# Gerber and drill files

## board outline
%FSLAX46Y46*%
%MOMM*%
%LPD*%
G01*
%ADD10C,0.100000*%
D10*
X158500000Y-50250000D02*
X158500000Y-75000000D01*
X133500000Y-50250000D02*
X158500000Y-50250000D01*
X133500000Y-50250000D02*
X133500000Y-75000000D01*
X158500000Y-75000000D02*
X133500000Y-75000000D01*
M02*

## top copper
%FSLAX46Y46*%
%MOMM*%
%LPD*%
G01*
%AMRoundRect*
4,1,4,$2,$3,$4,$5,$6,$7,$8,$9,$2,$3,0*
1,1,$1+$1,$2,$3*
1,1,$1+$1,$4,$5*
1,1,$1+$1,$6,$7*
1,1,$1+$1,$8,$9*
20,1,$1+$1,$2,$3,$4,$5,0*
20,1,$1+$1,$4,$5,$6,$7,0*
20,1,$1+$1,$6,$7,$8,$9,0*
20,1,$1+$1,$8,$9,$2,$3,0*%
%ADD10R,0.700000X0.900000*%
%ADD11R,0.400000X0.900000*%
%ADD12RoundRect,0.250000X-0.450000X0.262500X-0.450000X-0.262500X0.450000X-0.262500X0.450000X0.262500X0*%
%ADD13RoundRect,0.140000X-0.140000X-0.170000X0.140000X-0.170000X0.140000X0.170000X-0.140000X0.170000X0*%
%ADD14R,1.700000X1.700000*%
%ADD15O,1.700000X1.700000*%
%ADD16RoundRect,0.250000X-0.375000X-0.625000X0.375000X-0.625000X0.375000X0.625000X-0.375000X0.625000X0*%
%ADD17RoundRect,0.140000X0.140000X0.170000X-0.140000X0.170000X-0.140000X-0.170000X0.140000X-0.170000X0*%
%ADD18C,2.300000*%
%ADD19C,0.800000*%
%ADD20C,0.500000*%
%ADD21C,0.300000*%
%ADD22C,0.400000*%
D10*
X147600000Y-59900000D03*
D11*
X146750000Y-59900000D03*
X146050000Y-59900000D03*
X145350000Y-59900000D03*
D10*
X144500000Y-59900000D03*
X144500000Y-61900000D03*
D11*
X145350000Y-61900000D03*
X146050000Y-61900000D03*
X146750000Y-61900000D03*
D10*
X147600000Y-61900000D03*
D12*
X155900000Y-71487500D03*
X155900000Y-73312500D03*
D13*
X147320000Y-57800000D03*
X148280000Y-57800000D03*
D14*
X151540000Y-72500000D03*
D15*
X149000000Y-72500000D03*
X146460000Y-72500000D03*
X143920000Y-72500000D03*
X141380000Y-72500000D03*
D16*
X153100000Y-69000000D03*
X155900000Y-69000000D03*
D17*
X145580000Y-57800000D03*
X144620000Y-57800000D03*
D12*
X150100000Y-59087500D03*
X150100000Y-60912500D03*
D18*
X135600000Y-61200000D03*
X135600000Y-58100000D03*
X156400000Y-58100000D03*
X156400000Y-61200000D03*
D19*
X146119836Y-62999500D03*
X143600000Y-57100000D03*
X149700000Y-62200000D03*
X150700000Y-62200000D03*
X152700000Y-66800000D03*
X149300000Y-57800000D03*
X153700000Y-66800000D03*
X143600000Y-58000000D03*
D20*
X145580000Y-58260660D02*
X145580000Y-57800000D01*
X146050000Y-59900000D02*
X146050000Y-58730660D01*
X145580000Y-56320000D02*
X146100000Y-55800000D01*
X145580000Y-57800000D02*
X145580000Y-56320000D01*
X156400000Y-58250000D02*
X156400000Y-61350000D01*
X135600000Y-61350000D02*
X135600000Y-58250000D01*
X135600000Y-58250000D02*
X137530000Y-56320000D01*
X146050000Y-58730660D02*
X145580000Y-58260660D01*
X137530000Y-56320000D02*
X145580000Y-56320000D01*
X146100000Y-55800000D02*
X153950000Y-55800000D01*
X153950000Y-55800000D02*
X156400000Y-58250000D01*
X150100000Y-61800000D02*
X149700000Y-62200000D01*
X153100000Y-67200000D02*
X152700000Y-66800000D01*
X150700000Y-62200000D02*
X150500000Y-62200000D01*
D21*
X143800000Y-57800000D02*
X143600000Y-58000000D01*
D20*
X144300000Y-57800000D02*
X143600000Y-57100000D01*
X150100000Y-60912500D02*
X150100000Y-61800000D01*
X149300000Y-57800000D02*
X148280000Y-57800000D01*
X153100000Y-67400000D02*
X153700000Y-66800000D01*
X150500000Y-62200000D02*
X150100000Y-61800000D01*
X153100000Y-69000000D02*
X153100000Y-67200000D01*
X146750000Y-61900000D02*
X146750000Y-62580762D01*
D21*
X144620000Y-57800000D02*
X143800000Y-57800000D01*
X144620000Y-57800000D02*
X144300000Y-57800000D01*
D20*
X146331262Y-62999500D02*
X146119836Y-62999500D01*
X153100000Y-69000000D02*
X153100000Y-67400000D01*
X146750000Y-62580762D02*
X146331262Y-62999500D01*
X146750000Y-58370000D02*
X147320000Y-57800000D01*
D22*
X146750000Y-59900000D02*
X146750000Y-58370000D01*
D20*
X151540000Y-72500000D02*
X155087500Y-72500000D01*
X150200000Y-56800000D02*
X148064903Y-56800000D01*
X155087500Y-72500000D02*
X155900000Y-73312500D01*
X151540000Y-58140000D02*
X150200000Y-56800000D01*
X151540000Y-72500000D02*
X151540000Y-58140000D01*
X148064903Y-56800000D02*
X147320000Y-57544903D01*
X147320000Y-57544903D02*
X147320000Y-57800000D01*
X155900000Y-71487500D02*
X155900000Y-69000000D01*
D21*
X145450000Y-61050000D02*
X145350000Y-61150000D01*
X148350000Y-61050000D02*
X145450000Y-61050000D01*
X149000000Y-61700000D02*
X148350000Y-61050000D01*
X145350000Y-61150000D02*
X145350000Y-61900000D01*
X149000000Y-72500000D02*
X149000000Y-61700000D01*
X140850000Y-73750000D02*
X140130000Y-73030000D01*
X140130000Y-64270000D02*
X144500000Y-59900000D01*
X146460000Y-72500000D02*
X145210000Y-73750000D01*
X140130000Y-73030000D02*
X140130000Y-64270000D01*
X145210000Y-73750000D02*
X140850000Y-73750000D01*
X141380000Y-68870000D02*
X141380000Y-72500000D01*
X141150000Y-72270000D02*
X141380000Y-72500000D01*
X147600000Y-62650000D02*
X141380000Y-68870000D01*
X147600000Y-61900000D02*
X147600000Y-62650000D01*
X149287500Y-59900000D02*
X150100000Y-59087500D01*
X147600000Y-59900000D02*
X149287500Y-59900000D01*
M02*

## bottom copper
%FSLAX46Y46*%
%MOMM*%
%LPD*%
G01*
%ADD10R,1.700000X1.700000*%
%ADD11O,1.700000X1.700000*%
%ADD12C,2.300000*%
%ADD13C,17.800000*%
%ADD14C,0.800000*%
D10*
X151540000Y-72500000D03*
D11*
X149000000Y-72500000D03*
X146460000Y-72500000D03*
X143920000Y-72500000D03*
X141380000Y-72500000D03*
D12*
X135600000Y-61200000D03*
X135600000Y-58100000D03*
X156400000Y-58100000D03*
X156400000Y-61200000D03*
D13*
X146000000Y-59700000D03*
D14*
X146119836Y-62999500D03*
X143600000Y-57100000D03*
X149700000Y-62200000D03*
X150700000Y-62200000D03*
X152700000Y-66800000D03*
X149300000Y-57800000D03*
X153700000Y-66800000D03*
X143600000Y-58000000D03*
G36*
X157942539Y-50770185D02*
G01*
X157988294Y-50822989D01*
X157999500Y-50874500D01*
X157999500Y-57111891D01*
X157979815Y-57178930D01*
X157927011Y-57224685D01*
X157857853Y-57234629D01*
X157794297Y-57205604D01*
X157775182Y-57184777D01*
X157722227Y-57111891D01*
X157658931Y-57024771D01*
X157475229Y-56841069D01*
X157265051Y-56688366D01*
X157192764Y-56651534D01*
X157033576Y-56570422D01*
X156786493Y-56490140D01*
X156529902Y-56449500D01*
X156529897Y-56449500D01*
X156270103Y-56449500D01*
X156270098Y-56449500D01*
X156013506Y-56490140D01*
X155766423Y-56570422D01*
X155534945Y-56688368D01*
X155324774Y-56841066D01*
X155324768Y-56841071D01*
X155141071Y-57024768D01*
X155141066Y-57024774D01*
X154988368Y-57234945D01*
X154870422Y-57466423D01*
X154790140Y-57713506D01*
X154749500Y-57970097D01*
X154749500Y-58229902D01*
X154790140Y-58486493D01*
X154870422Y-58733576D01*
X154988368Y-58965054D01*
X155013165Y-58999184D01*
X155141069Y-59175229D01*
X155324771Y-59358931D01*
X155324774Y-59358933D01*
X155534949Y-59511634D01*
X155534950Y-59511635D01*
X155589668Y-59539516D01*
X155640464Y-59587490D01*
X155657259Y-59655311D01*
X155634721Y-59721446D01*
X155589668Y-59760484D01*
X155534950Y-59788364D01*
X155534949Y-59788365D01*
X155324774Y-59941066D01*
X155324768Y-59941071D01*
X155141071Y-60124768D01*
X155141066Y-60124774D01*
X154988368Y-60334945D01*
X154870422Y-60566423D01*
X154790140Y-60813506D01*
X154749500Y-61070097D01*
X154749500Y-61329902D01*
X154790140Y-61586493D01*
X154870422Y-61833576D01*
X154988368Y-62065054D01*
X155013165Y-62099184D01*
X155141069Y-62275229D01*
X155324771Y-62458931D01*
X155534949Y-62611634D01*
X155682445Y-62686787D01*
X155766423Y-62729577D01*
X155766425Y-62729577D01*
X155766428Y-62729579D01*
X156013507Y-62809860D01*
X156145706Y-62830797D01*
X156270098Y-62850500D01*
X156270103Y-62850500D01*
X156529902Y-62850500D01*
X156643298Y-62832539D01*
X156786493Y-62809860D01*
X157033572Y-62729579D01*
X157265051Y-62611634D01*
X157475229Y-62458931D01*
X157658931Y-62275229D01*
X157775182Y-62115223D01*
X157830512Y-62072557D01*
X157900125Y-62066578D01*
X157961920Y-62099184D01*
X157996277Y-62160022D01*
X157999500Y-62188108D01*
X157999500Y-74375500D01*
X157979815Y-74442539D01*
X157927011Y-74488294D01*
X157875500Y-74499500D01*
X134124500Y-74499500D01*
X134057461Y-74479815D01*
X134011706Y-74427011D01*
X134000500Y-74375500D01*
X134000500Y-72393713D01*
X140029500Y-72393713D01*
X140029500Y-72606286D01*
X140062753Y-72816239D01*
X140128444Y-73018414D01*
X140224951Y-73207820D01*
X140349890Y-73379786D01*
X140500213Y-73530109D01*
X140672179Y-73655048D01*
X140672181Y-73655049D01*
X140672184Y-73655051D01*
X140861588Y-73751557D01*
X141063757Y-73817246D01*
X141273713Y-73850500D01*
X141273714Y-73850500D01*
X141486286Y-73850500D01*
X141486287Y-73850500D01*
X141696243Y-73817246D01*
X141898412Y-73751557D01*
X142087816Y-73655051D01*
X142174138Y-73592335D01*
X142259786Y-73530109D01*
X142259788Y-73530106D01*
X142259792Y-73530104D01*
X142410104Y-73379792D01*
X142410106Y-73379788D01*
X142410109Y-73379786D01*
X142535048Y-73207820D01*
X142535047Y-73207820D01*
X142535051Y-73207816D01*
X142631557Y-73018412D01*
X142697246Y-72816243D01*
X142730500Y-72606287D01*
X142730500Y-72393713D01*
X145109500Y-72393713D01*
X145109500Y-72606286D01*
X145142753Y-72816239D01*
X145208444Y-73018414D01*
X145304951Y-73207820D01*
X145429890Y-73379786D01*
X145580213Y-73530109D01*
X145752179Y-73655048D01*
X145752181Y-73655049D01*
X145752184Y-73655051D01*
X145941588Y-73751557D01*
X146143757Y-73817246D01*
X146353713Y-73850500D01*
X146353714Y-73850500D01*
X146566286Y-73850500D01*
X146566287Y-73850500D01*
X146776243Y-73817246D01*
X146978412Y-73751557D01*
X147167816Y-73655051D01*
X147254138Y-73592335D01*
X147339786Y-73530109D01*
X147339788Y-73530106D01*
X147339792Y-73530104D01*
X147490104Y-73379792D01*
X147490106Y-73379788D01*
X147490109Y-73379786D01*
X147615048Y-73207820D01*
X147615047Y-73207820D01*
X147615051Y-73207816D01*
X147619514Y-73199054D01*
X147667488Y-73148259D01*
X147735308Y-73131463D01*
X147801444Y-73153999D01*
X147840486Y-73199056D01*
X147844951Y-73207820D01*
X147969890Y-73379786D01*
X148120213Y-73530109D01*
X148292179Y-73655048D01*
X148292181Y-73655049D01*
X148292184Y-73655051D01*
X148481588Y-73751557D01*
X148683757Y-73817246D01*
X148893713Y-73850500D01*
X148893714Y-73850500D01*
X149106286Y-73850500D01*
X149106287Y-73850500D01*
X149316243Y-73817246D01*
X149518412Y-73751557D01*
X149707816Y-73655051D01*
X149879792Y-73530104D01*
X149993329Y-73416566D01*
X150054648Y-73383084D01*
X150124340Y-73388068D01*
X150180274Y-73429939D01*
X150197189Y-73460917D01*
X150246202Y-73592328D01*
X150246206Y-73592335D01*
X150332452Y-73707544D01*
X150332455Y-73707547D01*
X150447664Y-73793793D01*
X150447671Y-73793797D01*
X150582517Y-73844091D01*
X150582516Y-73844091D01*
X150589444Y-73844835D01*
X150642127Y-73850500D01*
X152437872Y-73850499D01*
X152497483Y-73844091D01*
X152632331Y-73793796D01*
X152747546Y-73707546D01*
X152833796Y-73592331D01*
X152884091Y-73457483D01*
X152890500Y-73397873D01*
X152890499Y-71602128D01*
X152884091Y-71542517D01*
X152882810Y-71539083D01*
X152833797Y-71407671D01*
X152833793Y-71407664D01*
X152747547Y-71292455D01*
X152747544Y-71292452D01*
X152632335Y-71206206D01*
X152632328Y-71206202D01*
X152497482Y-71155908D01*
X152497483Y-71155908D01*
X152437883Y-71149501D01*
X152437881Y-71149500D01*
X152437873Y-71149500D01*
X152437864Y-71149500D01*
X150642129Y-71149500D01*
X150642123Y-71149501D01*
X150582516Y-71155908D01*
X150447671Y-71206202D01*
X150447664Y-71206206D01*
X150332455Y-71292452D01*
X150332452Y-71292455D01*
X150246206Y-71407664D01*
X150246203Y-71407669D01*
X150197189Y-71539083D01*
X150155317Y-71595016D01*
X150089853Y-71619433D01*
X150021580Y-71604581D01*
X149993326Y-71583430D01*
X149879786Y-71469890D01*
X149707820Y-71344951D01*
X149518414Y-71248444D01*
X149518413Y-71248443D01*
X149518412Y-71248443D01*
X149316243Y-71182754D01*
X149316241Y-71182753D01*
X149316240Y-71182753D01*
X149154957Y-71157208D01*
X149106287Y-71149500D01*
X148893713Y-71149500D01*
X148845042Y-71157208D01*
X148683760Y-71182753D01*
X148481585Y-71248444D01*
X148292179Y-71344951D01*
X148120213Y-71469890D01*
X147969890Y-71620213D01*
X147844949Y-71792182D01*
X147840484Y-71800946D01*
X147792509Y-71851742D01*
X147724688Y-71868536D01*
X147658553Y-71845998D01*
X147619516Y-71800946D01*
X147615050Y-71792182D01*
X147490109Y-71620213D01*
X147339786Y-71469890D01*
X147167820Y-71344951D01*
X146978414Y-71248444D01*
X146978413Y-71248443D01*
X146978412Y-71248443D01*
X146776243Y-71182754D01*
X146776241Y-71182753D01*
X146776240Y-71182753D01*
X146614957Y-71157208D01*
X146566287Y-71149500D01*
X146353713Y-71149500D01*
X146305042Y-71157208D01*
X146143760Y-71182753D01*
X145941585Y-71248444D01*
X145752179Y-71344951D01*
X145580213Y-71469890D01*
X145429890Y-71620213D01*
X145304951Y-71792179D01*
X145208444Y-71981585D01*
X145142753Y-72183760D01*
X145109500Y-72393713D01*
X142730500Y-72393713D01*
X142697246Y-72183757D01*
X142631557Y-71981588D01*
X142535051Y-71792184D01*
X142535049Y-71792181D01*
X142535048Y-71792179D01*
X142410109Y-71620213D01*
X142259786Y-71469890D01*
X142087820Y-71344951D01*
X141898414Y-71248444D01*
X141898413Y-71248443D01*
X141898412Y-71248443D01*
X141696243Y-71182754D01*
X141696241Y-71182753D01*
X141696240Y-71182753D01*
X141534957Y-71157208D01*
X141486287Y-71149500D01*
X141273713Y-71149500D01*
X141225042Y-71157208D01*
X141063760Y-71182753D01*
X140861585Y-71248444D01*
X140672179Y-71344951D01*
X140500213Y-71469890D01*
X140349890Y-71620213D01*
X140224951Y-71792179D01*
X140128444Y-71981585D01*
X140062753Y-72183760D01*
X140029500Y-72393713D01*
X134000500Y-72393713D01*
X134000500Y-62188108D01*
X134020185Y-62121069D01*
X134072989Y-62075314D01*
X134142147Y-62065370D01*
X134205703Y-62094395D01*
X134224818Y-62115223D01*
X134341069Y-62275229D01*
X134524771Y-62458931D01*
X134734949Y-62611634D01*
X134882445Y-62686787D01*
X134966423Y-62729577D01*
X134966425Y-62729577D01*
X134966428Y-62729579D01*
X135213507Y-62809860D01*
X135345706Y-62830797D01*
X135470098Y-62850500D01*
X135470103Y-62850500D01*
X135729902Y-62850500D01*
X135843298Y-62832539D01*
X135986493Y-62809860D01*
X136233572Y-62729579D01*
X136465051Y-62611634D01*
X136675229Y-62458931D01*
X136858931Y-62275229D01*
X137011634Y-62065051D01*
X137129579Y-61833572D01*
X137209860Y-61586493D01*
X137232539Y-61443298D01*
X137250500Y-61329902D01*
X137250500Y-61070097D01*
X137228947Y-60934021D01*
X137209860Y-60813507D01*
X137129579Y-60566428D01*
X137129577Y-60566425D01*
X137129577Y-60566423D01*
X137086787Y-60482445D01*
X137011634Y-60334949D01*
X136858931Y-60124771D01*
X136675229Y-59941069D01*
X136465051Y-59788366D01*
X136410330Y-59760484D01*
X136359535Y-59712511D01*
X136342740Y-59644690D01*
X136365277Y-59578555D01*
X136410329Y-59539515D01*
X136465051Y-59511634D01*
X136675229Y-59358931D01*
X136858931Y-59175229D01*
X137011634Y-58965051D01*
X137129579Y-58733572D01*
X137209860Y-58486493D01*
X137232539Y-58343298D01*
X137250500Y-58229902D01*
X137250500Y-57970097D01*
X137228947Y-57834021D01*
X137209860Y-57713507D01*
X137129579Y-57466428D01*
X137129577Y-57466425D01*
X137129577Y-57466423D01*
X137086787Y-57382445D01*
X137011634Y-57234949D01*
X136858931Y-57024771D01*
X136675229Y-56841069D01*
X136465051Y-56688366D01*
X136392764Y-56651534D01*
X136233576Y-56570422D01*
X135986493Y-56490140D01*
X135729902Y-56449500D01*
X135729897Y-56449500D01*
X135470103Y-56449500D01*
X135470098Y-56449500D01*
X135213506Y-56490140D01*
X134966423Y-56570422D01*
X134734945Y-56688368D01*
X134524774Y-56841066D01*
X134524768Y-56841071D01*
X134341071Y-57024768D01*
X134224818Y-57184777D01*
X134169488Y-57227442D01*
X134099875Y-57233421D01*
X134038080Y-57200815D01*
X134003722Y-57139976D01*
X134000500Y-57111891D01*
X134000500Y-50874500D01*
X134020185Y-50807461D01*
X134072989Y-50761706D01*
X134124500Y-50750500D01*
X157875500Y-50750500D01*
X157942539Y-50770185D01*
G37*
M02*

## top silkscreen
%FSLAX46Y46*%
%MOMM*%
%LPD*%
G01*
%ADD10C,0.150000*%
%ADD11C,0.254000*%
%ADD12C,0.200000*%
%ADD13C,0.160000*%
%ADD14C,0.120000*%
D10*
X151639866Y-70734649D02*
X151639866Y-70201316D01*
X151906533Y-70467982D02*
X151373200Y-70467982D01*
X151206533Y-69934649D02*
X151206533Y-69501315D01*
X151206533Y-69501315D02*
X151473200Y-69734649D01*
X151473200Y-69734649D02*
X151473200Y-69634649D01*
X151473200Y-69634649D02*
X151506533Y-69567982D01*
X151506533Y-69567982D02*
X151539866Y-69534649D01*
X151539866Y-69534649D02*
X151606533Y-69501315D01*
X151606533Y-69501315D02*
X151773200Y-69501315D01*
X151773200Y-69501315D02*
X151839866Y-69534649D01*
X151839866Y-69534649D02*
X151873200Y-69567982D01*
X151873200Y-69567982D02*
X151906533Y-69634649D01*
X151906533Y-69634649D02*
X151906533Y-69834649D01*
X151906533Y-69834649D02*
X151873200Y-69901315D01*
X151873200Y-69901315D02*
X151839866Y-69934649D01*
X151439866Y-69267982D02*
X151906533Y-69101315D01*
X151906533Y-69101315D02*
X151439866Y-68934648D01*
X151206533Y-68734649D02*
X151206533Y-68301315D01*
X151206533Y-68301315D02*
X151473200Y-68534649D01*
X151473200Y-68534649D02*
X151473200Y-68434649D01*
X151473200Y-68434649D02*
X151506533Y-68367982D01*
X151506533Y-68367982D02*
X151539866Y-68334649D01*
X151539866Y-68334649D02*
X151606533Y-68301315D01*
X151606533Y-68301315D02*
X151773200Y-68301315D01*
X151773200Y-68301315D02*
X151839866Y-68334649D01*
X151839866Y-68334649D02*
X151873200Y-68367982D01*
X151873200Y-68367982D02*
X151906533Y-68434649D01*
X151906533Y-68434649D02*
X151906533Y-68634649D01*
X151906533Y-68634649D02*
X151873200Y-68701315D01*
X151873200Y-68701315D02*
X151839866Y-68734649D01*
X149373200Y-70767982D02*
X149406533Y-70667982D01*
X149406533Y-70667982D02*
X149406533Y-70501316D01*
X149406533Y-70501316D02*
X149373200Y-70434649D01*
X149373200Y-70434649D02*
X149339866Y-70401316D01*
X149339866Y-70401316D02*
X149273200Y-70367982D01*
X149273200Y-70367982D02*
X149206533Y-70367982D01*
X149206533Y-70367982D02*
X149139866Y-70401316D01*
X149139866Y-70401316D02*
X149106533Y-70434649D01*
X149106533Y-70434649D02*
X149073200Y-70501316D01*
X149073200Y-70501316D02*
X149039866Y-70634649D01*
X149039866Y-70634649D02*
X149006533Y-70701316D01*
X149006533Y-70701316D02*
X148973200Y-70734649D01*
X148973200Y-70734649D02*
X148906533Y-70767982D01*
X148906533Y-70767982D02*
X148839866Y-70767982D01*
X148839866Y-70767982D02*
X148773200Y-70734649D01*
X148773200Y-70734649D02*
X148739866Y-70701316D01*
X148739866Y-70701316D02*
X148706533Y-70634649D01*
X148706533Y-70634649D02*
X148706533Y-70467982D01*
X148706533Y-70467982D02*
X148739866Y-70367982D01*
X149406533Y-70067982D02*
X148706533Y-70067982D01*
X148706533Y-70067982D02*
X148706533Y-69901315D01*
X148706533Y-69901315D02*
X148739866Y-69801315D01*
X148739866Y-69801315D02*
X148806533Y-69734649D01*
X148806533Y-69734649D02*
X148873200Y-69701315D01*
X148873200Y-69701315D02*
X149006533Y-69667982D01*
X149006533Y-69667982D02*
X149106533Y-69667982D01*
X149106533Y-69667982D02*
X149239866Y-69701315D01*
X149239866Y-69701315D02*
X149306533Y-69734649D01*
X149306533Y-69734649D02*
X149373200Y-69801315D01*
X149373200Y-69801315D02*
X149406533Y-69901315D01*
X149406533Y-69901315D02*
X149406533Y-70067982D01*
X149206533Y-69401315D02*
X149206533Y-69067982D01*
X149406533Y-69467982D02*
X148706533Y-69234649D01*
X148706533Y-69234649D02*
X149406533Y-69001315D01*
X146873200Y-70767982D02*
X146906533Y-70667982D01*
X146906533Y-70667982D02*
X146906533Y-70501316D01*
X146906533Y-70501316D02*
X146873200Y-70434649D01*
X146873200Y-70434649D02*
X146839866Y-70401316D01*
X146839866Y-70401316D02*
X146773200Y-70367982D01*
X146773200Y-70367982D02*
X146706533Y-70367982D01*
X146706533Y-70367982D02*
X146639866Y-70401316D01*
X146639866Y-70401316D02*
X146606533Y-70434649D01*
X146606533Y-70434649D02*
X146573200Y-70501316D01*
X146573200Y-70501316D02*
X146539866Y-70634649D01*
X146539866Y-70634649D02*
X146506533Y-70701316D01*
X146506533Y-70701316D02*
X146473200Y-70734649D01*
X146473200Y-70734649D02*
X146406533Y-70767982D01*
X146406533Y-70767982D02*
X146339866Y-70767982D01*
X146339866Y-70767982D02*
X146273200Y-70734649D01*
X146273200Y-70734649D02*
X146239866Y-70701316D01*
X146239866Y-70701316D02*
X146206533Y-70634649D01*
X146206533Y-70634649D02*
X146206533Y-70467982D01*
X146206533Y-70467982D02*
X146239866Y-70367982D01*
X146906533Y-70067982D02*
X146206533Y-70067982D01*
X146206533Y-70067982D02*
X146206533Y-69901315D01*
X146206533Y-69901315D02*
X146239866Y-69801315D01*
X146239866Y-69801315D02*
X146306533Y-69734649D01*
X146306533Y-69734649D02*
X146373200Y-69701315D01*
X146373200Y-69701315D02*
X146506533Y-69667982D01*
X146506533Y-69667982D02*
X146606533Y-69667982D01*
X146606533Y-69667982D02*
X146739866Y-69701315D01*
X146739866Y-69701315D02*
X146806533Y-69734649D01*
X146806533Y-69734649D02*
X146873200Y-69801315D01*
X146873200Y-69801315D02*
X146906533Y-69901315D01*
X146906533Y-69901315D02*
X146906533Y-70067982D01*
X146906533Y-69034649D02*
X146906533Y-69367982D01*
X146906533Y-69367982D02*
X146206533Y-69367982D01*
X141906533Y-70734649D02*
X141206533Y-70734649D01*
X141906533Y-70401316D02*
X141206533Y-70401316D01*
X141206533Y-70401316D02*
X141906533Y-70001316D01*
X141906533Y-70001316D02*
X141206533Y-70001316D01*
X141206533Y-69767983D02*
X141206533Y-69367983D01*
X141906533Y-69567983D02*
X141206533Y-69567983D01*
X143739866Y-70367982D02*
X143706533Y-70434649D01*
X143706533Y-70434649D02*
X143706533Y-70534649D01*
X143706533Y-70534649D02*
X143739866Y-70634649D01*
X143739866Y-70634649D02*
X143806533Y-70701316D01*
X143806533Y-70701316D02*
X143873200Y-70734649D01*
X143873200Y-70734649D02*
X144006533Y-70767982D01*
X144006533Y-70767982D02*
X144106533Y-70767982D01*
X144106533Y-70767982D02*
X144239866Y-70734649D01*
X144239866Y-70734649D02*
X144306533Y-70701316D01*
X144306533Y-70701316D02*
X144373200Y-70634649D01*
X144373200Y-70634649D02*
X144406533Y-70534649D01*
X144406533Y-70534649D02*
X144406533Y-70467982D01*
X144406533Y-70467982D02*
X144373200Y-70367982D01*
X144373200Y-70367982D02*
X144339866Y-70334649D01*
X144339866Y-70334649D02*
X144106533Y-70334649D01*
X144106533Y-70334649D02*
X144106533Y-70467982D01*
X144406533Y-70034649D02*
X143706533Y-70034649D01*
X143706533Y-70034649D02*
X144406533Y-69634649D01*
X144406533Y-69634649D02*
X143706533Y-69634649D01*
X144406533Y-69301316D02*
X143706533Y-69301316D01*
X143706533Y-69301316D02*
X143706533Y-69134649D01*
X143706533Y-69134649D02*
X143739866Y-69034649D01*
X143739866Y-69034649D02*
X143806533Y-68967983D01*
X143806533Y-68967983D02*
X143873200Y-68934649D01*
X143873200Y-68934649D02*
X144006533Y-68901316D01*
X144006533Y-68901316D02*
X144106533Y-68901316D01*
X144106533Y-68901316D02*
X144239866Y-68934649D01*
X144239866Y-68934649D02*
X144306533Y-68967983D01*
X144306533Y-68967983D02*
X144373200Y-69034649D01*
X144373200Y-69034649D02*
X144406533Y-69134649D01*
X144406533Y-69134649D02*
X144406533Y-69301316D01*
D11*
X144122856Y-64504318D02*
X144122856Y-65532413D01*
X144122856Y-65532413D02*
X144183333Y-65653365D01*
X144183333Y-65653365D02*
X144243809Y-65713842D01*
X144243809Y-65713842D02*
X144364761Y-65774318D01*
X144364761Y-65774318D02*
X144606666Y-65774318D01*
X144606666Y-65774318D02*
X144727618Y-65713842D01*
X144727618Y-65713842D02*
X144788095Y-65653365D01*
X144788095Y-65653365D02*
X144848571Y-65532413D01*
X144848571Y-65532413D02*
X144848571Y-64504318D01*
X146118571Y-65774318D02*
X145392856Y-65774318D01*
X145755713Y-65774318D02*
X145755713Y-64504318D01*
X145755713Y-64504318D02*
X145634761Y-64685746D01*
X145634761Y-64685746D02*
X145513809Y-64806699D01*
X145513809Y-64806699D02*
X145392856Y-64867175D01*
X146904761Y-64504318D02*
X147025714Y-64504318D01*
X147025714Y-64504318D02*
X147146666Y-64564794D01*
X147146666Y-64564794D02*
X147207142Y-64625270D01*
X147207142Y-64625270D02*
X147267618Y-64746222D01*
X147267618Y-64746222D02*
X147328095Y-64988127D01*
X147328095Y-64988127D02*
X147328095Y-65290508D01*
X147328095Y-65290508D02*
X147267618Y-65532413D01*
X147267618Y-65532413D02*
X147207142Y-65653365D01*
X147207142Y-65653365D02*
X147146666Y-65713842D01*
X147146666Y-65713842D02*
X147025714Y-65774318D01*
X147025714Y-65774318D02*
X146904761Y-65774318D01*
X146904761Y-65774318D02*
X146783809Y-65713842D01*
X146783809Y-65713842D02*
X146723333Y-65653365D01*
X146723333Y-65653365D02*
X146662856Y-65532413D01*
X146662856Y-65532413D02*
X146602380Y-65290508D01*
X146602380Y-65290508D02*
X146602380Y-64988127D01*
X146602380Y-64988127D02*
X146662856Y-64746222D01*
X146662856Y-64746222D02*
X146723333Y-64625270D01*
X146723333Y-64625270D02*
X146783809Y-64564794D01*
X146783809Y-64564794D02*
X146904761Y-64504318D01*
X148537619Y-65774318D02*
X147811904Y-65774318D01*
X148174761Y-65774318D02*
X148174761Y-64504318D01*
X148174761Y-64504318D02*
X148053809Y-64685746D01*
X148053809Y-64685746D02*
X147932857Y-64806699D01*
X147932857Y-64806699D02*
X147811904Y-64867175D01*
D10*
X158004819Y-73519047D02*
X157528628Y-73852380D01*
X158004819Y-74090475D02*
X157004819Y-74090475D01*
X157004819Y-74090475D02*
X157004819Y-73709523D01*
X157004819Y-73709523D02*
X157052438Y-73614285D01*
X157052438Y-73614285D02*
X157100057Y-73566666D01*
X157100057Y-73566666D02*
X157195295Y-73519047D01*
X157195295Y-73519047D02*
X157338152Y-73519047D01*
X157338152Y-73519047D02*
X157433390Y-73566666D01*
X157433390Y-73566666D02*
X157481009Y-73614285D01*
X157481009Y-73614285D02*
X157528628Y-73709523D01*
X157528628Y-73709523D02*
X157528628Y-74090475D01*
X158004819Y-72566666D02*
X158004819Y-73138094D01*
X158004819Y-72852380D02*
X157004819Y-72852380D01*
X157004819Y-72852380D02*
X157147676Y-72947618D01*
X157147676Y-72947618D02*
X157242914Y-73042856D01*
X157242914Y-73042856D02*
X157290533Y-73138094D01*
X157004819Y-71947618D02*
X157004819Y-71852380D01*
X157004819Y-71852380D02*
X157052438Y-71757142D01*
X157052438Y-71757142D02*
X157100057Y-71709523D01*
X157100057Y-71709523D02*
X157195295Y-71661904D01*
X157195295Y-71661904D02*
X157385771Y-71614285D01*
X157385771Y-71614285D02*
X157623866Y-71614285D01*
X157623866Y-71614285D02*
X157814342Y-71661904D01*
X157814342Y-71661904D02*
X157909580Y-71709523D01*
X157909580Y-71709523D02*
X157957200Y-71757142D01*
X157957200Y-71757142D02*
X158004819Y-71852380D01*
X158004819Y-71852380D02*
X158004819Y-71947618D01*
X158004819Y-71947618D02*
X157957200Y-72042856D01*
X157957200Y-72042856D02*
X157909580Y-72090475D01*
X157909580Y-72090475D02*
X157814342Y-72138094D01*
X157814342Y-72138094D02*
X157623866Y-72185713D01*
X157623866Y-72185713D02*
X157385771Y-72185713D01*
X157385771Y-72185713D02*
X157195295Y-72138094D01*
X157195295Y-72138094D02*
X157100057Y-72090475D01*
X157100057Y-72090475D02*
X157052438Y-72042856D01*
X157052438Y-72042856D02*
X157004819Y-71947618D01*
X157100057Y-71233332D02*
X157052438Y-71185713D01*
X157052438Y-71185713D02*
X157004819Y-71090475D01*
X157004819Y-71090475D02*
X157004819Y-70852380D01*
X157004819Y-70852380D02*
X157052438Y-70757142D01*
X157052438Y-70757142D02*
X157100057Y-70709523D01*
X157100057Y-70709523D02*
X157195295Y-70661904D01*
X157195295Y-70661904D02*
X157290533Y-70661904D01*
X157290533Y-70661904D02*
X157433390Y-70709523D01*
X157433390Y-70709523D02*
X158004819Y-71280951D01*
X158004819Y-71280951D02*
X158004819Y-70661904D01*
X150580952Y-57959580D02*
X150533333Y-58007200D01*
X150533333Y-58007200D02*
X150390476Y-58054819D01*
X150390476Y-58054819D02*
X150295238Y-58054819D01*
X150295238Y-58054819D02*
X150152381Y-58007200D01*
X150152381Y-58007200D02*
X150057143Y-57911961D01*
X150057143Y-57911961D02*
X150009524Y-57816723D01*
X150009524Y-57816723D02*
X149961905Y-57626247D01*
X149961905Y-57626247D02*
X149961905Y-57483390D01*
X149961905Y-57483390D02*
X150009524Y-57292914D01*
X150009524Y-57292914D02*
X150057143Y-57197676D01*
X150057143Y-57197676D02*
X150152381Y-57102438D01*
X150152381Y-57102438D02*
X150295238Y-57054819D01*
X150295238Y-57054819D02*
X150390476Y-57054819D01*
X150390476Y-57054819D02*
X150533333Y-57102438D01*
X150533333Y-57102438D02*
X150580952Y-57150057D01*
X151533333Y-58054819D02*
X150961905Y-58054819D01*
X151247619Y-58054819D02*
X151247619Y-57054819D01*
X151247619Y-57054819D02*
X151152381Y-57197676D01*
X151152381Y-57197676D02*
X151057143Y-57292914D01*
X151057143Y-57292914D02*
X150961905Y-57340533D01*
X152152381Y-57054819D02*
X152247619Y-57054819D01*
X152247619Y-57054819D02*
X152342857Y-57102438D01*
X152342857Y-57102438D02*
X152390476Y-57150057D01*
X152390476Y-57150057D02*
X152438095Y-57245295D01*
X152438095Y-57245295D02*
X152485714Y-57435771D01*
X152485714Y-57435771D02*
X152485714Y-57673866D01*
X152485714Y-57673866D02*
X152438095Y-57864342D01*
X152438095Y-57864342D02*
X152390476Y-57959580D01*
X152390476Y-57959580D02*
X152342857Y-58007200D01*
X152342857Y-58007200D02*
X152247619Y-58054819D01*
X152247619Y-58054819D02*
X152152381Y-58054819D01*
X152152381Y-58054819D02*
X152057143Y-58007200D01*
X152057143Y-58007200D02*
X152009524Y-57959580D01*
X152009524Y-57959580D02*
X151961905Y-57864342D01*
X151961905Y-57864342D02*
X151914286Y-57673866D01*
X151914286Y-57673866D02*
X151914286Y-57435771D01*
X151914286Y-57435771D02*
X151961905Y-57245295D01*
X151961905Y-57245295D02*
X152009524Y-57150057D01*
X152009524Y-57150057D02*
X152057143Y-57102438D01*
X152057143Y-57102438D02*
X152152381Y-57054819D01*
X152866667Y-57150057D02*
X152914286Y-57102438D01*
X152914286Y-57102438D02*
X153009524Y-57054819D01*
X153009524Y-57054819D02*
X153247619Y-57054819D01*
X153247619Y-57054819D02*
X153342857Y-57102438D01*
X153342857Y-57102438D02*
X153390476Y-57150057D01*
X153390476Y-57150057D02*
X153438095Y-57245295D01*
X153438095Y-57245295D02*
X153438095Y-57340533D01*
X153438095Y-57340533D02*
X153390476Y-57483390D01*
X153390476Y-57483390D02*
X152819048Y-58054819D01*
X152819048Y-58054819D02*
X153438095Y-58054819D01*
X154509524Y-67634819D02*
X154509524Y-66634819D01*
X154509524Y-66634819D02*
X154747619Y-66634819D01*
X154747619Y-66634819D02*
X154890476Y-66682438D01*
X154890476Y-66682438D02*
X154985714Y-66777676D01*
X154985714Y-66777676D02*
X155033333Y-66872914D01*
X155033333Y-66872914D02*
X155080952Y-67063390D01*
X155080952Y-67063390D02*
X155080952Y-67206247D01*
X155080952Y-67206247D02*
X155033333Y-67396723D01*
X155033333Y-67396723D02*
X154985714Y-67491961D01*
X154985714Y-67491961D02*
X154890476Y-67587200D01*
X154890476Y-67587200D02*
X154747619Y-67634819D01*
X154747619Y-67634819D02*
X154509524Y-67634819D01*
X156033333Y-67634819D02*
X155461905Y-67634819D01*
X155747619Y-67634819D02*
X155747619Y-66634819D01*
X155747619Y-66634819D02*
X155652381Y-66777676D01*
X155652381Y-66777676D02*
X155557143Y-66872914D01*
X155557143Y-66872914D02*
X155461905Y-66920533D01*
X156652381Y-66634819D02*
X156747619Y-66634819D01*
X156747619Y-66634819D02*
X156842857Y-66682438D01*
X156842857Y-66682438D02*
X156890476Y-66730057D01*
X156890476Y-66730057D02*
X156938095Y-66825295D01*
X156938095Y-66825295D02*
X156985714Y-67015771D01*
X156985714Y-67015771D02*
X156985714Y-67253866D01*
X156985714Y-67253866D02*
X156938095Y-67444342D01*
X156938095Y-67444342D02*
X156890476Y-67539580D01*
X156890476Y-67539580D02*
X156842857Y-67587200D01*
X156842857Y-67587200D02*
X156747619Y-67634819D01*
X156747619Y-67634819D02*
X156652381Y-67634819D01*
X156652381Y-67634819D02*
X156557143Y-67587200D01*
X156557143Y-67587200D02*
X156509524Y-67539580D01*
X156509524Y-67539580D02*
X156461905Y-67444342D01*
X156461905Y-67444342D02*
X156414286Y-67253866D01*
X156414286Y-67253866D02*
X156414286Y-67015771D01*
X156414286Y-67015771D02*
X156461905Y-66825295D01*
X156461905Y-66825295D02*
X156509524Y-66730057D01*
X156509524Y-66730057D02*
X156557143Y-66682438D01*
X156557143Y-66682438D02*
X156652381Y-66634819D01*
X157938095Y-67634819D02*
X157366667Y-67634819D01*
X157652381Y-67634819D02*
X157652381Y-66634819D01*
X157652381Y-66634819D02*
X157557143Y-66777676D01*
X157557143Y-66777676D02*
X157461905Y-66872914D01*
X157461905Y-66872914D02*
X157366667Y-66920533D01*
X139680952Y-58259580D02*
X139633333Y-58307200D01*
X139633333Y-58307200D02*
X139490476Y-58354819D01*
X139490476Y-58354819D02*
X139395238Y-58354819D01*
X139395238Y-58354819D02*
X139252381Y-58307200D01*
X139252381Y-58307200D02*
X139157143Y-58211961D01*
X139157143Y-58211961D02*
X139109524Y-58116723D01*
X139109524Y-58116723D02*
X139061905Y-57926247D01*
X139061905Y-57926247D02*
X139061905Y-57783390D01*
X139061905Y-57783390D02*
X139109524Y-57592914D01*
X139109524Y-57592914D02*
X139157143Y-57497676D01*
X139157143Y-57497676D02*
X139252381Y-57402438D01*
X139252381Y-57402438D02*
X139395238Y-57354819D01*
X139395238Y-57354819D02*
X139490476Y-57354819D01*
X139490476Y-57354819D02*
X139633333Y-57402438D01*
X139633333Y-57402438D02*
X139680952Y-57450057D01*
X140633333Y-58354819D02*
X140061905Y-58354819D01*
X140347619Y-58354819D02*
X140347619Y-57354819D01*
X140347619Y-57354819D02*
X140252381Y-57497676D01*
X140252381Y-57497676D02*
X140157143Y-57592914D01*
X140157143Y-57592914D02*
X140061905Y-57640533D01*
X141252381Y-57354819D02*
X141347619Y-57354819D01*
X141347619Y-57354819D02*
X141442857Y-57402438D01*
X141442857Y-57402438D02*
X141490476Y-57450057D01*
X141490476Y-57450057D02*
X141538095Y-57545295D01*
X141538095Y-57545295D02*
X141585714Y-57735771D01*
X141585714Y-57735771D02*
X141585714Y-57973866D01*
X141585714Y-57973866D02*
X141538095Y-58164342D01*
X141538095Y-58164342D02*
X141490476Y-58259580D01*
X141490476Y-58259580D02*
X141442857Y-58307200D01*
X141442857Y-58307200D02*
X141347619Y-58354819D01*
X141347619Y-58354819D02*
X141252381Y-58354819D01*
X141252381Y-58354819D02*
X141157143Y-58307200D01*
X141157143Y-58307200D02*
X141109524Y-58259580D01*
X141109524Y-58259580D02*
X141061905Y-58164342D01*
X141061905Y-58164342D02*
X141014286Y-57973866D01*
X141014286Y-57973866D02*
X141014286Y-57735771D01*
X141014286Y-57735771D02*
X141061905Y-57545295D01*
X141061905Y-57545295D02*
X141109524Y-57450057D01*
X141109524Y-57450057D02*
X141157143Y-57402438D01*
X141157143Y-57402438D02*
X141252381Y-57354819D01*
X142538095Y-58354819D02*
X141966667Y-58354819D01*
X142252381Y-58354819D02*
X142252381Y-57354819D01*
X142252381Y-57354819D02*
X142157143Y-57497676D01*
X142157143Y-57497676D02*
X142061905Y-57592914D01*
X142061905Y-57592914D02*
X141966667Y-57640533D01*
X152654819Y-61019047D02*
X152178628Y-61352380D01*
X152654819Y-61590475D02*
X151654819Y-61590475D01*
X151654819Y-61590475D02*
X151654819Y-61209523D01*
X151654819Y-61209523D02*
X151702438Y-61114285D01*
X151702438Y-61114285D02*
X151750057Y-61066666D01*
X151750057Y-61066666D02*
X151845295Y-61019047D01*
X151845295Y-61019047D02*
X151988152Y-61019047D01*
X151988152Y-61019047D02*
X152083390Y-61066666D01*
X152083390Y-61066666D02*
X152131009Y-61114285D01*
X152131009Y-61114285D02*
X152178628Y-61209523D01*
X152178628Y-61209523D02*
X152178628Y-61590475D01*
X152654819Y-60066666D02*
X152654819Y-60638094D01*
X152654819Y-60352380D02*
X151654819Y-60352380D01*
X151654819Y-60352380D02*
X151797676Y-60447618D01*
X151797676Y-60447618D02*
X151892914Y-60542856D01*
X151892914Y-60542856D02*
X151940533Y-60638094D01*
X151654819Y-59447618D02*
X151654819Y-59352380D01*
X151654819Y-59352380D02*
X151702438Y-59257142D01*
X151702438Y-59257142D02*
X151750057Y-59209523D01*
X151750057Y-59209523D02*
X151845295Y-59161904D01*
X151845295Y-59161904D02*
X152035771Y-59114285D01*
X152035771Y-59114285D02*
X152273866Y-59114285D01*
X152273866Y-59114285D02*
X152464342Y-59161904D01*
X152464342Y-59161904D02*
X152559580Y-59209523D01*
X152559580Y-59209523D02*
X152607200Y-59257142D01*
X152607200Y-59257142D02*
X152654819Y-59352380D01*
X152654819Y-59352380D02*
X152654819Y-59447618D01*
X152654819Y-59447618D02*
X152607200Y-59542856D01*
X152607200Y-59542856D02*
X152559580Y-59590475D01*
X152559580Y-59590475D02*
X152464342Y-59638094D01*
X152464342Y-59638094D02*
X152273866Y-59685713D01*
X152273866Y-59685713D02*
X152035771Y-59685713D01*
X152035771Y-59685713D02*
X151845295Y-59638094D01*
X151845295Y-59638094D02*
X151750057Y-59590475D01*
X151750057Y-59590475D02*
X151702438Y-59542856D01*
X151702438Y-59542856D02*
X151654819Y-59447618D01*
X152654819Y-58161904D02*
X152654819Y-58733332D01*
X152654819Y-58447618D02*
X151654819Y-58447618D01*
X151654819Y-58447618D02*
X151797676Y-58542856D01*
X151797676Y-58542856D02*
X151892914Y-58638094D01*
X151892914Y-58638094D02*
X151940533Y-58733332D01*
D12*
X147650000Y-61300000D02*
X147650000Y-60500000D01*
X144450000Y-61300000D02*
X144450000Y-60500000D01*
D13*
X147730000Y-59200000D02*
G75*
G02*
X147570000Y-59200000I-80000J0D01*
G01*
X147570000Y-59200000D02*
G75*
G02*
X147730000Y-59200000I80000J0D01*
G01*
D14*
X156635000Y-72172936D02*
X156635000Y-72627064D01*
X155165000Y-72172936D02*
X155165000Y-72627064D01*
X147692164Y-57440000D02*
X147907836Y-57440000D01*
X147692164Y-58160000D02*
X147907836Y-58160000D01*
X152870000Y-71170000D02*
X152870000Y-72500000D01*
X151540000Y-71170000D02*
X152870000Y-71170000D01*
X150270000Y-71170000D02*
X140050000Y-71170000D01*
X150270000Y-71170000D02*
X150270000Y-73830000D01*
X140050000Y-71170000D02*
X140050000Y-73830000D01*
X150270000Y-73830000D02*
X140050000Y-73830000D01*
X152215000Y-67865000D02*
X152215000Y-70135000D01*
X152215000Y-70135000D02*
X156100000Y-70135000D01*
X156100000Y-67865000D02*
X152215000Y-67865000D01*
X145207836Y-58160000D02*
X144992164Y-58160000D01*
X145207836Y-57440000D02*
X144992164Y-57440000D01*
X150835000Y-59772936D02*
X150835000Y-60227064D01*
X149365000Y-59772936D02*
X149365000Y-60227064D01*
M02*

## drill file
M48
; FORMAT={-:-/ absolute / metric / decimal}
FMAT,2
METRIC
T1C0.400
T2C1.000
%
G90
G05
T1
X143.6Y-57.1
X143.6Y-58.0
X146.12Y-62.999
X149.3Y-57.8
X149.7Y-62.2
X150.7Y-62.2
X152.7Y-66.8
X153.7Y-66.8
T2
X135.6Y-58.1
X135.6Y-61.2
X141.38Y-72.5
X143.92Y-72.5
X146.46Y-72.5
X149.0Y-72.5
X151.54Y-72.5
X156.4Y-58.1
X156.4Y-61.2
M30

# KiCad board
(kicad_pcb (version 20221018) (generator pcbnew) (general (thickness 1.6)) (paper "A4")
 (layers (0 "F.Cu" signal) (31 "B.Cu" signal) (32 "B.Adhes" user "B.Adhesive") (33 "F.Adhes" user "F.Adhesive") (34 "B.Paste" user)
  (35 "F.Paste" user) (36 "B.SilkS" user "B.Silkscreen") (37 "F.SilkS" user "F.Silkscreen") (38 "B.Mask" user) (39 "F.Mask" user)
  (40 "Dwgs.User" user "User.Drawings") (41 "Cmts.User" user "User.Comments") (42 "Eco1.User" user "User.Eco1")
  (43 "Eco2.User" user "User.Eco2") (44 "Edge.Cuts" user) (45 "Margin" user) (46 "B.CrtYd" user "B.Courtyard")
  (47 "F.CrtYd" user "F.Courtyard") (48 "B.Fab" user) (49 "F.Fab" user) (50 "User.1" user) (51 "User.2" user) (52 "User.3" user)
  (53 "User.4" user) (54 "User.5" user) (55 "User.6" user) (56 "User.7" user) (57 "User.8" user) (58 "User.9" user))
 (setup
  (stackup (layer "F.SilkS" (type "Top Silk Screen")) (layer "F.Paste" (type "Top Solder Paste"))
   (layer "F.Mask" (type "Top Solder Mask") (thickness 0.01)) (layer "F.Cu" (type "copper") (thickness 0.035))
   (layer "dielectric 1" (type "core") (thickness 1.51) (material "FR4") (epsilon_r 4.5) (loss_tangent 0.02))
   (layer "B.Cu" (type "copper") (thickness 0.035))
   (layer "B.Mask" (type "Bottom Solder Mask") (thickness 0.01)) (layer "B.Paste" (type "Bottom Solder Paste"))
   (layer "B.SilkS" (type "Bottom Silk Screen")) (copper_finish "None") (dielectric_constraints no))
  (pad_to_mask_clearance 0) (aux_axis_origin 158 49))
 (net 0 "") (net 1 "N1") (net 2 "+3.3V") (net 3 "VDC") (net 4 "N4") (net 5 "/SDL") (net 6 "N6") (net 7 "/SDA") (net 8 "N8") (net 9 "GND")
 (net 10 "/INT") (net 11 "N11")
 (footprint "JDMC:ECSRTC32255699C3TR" (layer "F.Cu") (at 146.05 60.9 180)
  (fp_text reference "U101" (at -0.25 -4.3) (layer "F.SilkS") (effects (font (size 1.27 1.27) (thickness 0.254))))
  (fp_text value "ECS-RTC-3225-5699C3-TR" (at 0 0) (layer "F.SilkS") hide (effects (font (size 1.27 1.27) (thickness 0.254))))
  (fp_line (start -1.6 -0.4) (end -1.6 0.4) (stroke (width 0.2) (type solid)) (layer "F.SilkS"))
  (fp_line (start 1.6 -0.4) (end 1.6 0.4) (stroke (width 0.2) (type solid)) (layer "F.SilkS"))
  (fp_circle (center -1.6 1.7) (end -1.5 1.7) (stroke (width 0.12) (type solid)) (fill solid) (layer "F.SilkS"))
  (pad "1" smd rect (at -1.55 1 180) (size 0.7 0.9) (layers "F.Cu" "F.Paste" "F.Mask") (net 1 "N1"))
  (pad "2" smd rect (at -0.7 1 180) (size 0.4 0.9) (layers "F.Cu" "F.Paste" "F.Mask") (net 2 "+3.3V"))
  (pad "3" smd rect (at 0 1 180) (size 0.4 0.9) (layers "F.Cu" "F.Paste" "F.Mask") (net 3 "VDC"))
  (pad "4" smd rect (at 0.7 1 180) (size 0.4 0.9) (layers "F.Cu" "F.Paste" "F.Mask") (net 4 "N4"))
  (pad "5" smd rect (at 1.55 1 180) (size 0.7 0.9) (layers "F.Cu" "F.Paste" "F.Mask") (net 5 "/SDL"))
  (pad "6" smd rect (at 1.55 -1 180) (size 0.7 0.9) (layers "F.Cu" "F.Paste" "F.Mask") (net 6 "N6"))
  (pad "7" smd rect (at 0.7 -1 180) (size 0.4 0.9) (layers "F.Cu" "F.Paste" "F.Mask") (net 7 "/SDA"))
  (pad "8" smd rect (at 0 -1 180) (size 0.4 0.9) (layers "F.Cu" "F.Paste" "F.Mask") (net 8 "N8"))
  (pad "9" smd rect (at -0.7 -1 180) (size 0.4 0.9) (layers "F.Cu" "F.Paste" "F.Mask") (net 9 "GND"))
  (pad "10" smd rect (at -1.55 -1 180) (size 0.7 0.9) (layers "F.Cu" "F.Paste" "F.Mask") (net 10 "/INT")))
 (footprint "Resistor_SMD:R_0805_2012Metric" (layer "F.Cu") (at 155.9 72.4 -90)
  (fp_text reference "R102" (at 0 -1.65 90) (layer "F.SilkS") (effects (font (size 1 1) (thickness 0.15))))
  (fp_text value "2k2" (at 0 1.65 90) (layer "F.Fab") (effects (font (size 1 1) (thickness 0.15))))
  (fp_line (start -0.227064 -0.735) (end 0.227064 -0.735) (stroke (width 0.12) (type solid)) (layer "F.SilkS"))
  (fp_line (start -0.227064 0.735) (end 0.227064 0.735) (stroke (width 0.12) (type solid)) (layer "F.SilkS"))
  (pad "1" smd roundrect (at -0.9125 0 270) (size 1.025 1.4) (layers "F.Cu" "F.Paste" "F.Mask") (roundrect_rratio 0.243902) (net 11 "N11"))
  (pad "2" smd roundrect (at 0.9125 0 270) (size 1.025 1.4) (layers "F.Cu" "F.Paste" "F.Mask") (roundrect_rratio 0.243902) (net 2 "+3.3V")))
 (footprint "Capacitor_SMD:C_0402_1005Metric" (layer "F.Cu") (at 147.8 57.8)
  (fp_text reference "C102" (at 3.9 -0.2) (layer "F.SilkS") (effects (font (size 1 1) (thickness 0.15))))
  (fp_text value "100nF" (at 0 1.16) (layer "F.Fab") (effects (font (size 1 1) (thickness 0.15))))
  (fp_line (start -0.107836 -0.36) (end 0.107836 -0.36) (stroke (width 0.12) (type solid)) (layer "F.SilkS"))
  (fp_line (start -0.107836 0.36) (end 0.107836 0.36) (stroke (width 0.12) (type solid)) (layer "F.SilkS"))
  (pad "1" smd roundrect (at -0.48 0) (size 0.56 0.62) (layers "F.Cu" "F.Paste" "F.Mask") (roundrect_rratio 0.25) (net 2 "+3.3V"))
  (pad "2" smd roundrect (at 0.48 0) (size 0.56 0.62) (layers "F.Cu" "F.Paste" "F.Mask") (roundrect_rratio 0.25) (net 9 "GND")))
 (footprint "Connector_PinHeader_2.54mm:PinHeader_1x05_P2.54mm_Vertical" (layer "F.Cu") (at 151.54 72.5 -90)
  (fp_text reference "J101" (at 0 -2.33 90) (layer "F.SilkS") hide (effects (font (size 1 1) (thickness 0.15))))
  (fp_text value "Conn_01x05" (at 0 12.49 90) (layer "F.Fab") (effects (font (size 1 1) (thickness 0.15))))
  (fp_line (start -1.33 -1.33) (end 0 -1.33) (stroke (width 0.12) (type solid)) (layer "F.SilkS"))
  (fp_line (start -1.33 0) (end -1.33 -1.33) (stroke (width 0.12) (type solid)) (layer "F.SilkS"))
  (fp_line (start -1.33 1.27) (end -1.33 11.49) (stroke (width 0.12) (type solid)) (layer "F.SilkS"))
  (fp_line (start -1.33 1.27) (end 1.33 1.27) (stroke (width 0.12) (type solid)) (layer "F.SilkS"))
  (fp_line (start -1.33 11.49) (end 1.33 11.49) (stroke (width 0.12) (type solid)) (layer "F.SilkS"))
  (fp_line (start 1.33 1.27) (end 1.33 11.49) (stroke (width 0.12) (type solid)) (layer "F.SilkS"))
  (pad "1" thru_hole rect (at 0 0 270) (size 1.7 1.7) (drill 1) (layers "*.Cu" "*.Mask") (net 2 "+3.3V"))
  (pad "2" thru_hole oval (at 0 2.54 270) (size 1.7 1.7) (drill 1) (layers "*.Cu" "*.Mask") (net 7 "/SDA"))
  (pad "3" thru_hole oval (at 0 5.08 270) (size 1.7 1.7) (drill 1) (layers "*.Cu" "*.Mask") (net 5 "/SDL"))
  (pad "4" thru_hole oval (at 0 7.62 270) (size 1.7 1.7) (drill 1) (layers "*.Cu" "*.Mask") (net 9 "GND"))
  (pad "5" thru_hole oval (at 0 10.16 270) (size 1.7 1.7) (drill 1) (layers "*.Cu" "*.Mask") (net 10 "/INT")))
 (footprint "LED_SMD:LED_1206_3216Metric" (layer "F.Cu") (at 154.5 69)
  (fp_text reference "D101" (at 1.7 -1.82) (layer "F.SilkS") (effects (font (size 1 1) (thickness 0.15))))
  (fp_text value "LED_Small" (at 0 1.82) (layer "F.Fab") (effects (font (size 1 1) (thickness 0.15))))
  (fp_line (start -2.285 -1.135) (end -2.285 1.135) (stroke (width 0.12) (type solid)) (layer "F.SilkS"))
  (fp_line (start -2.285 1.135) (end 1.6 1.135) (stroke (width 0.12) (type solid)) (layer "F.SilkS"))
  (fp_line (start 1.6 -1.135) (end -2.285 -1.135) (stroke (width 0.12) (type solid)) (layer "F.SilkS"))
  (pad "1" smd roundrect (at -1.4 0) (size 1.25 1.75) (layers "F.Cu" "F.Paste" "F.Mask") (roundrect_rratio 0.2) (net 9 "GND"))
  (pad "2" smd roundrect (at 1.4 0) (size 1.25 1.75) (layers "F.Cu" "F.Paste" "F.Mask") (roundrect_rratio 0.2) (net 11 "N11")))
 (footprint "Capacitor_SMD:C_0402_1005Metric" (layer "F.Cu") (at 145.1 57.8 180)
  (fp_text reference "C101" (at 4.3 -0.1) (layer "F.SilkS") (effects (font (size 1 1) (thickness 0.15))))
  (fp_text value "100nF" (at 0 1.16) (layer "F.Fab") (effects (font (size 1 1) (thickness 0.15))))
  (fp_line (start -0.107836 -0.36) (end 0.107836 -0.36) (stroke (width 0.12) (type solid)) (layer "F.SilkS"))
  (fp_line (start -0.107836 0.36) (end 0.107836 0.36) (stroke (width 0.12) (type solid)) (layer "F.SilkS"))
  (pad "1" smd roundrect (at -0.48 0 180) (size 0.56 0.62) (layers "F.Cu" "F.Paste" "F.Mask") (roundrect_rratio 0.25) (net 3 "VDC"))
  (pad "2" smd roundrect (at 0.48 0 180) (size 0.56 0.62) (layers "F.Cu" "F.Paste" "F.Mask") (roundrect_rratio 0.25) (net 9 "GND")))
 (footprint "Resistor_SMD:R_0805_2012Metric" (layer "F.Cu") (at 150.1 60 -90)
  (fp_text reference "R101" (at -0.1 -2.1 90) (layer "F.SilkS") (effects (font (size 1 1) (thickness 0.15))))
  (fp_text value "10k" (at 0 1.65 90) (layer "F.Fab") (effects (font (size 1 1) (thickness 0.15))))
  (fp_line (start -0.227064 -0.735) (end 0.227064 -0.735) (stroke (width 0.12) (type solid)) (layer "F.SilkS"))
  (fp_line (start -0.227064 0.735) (end 0.227064 0.735) (stroke (width 0.12) (type solid)) (layer "F.SilkS"))
  (pad "1" smd roundrect (at -0.9125 0 270) (size 1.025 1.4) (layers "F.Cu" "F.Paste" "F.Mask") (roundrect_rratio 0.243902) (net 1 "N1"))
  (pad "2" smd roundrect (at 0.9125 0 270) (size 1.025 1.4) (layers "F.Cu" "F.Paste" "F.Mask") (roundrect_rratio 0.243902) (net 9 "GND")))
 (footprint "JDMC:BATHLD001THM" (layer "B.Cu") (at 146 59.7)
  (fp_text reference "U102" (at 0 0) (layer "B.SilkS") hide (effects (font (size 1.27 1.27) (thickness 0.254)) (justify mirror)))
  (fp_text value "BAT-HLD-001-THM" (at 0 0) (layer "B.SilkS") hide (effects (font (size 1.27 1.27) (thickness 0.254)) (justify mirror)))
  (pad "1" thru_hole circle (at -10.4 1.5) (size 2.3 2.3) (drill 1) (layers "*.Cu" "*.Mask") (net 3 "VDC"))
  (pad "2" thru_hole circle (at -10.4 -1.6) (size 2.3 2.3) (drill 1) (layers "*.Cu" "*.Mask") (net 3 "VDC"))
  (pad "3" thru_hole circle (at 10.4 -1.6) (size 2.3 2.3) (drill 1) (layers "*.Cu" "*.Mask") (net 3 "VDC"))
  (pad "4" thru_hole circle (at 10.4 1.5) (size 2.3 2.3) (drill 1) (layers "*.Cu" "*.Mask") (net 3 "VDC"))
  (pad "5" smd circle (at 0 0 270) (size 17.8 17.8) (layers "B.Cu" "B.Paste" "B.Mask") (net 9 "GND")))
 (gr_line (start 158.5 50.25) (end 158.5 75) (stroke (width 0.1) (type default)) (layer "Edge.Cuts"))
 (gr_line (start 133.5 50.25) (end 158.5 50.25) (stroke (width 0.1) (type default)) (layer "Edge.Cuts"))
 (gr_line (start 133.5 50.25) (end 133.5 75) (stroke (width 0.1) (type default)) (layer "Edge.Cuts"))
 (gr_line (start 158.5 75) (end 133.5 75) (stroke (width 0.1) (type default)) (layer "Edge.Cuts"))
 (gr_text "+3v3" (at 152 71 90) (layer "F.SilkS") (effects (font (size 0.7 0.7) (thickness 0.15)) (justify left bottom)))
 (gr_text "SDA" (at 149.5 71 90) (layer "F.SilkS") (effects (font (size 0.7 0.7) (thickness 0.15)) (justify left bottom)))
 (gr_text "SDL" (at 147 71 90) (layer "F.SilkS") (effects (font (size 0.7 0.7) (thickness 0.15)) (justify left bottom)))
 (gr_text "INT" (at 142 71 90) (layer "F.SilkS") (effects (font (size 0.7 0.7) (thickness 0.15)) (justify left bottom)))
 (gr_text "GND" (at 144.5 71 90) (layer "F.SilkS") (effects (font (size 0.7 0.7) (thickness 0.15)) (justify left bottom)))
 (segment (start 145.58 58.26066) (end 145.58 57.8) (width 0.5) (layer "F.Cu") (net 3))
 (segment (start 146.05 59.9) (end 146.05 58.73066) (width 0.5) (layer "F.Cu") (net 3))
 (segment (start 145.58 56.32) (end 146.1 55.8) (width 0.5) (layer "F.Cu") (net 3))
 (segment (start 145.58 57.8) (end 145.58 56.32) (width 0.5) (layer "F.Cu") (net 3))
 (segment (start 156.4 58.25) (end 156.4 61.35) (width 0.5) (layer "F.Cu") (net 3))
 (segment (start 135.6 61.35) (end 135.6 58.25) (width 0.5) (layer "F.Cu") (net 3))
 (segment (start 135.6 58.25) (end 137.53 56.32) (width 0.5) (layer "F.Cu") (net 3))
 (segment (start 146.05 58.73066) (end 145.58 58.26066) (width 0.5) (layer "F.Cu") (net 3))
 (segment (start 137.53 56.32) (end 145.58 56.32) (width 0.5) (layer "F.Cu") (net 3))
 (segment (start 146.1 55.8) (end 153.95 55.8) (width 0.5) (layer "F.Cu") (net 3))
 (segment (start 153.95 55.8) (end 156.4 58.25) (width 0.5) (layer "F.Cu") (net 3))
 (segment (start 150.1 61.8) (end 149.7 62.2) (width 0.5) (layer "F.Cu") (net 9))
 (segment (start 153.1 67.2) (end 152.7 66.8) (width 0.5) (layer "F.Cu") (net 9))
 (segment (start 150.7 62.2) (end 150.5 62.2) (width 0.5) (layer "F.Cu") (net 9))
 (segment (start 143.8 57.8) (end 143.6 58) (width 0.3) (layer "F.Cu") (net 9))
 (segment (start 144.3 57.8) (end 143.6 57.1) (width 0.5) (layer "F.Cu") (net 9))
 (segment (start 150.1 60.9125) (end 150.1 61.8) (width 0.5) (layer "F.Cu") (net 9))
 (segment (start 149.3 57.8) (end 148.28 57.8) (width 0.5) (layer "F.Cu") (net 9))
 (segment (start 153.1 67.4) (end 153.7 66.8) (width 0.5) (layer "F.Cu") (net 9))
 (segment (start 150.5 62.2) (end 150.1 61.8) (width 0.5) (layer "F.Cu") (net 9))
 (segment (start 153.1 69) (end 153.1 67.2) (width 0.5) (layer "F.Cu") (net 9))
 (segment (start 146.75 61.9) (end 146.75 62.580762) (width 0.5) (layer "F.Cu") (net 9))
 (segment (start 144.62 57.8) (end 143.8 57.8) (width 0.3) (layer "F.Cu") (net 9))
 (segment (start 144.62 57.8) (end 144.3 57.8) (width 0.3) (layer "F.Cu") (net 9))
 (segment (start 146.331262 62.9995) (end 146.119836 62.9995) (width 0.5) (layer "F.Cu") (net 9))
 (segment (start 153.1 69) (end 153.1 67.4) (width 0.5) (layer "F.Cu") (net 9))
 (segment (start 146.75 62.580762) (end 146.331262 62.9995) (width 0.5) (layer "F.Cu") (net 9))
 (via (at 146.119836 62.9995) (size 0.8) (drill 0.4) (layers "F.Cu" "B.Cu") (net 9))
 (via (at 143.6 57.1) (size 0.8) (drill 0.4) (layers "F.Cu" "B.Cu") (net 9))
 (via (at 149.7 62.2) (size 0.8) (drill 0.4) (layers "F.Cu" "B.Cu") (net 9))
 (via (at 150.7 62.2) (size 0.8) (drill 0.4) (layers "F.Cu" "B.Cu") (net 9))
 (via (at 152.7 66.8) (size 0.8) (drill 0.4) (layers "F.Cu" "B.Cu") (free) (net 9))
 (via (at 149.3 57.8) (size 0.8) (drill 0.4) (layers "F.Cu" "B.Cu") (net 9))
 (via (at 153.7 66.8) (size 0.8) (drill 0.4) (layers "F.Cu" "B.Cu") (free) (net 9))
 (via (at 143.6 58) (size 0.8) (drill 0.4) (layers "F.Cu" "B.Cu") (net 9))
 (segment (start 146.75 58.37) (end 147.32 57.8) (width 0.5) (layer "F.Cu") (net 2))
 (segment (start 146.75 59.9) (end 146.75 58.37) (width 0.4) (layer "F.Cu") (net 2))
 (segment (start 151.54 72.5) (end 155.0875 72.5) (width 0.5) (layer "F.Cu") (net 2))
 (segment (start 150.2 56.8) (end 148.064903 56.8) (width 0.5) (layer "F.Cu") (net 2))
 (segment (start 155.0875 72.5) (end 155.9 73.3125) (width 0.5) (layer "F.Cu") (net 2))
 (segment (start 151.54 58.14) (end 150.2 56.8) (width 0.5) (layer "F.Cu") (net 2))
 (segment (start 151.54 72.5) (end 151.54 58.14) (width 0.5) (layer "F.Cu") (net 2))
 (segment (start 148.064903 56.8) (end 147.32 57.544903) (width 0.5) (layer "F.Cu") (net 2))
 (segment (start 147.32 57.544903) (end 147.32 57.8) (width 0.5) (layer "F.Cu") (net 2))
 (segment (start 155.9 71.4875) (end 155.9 69) (width 0.5) (layer "F.Cu") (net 11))
 (segment (start 145.45 61.05) (end 145.35 61.15) (width 0.3) (layer "F.Cu") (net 7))
 (segment (start 148.35 61.05) (end 145.45 61.05) (width 0.3) (layer "F.Cu") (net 7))
 (segment (start 149 61.7) (end 148.35 61.05) (width 0.3) (layer "F.Cu") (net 7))
 (segment (start 145.35 61.15) (end 145.35 61.9) (width 0.3) (layer "F.Cu") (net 7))
 (segment (start 149 72.5) (end 149 61.7) (width 0.3) (layer "F.Cu") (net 7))
 (segment (start 140.85 73.75) (end 140.13 73.03) (width 0.3) (layer "F.Cu") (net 5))
 (segment (start 140.13 64.27) (end 144.5 59.9) (width 0.3) (layer "F.Cu") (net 5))
 (segment (start 146.46 72.5) (end 145.21 73.75) (width 0.3) (layer "F.Cu") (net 5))
 (segment (start 140.13 73.03) (end 140.13 64.27) (width 0.3) (layer "F.Cu") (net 5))
 (segment (start 145.21 73.75) (end 140.85 73.75) (width 0.3) (layer "F.Cu") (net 5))
 (segment (start 141.38 68.87) (end 141.38 72.5) (width 0.3) (layer "F.Cu") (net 10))
 (segment (start 141.15 72.27) (end 141.38 72.5) (width 0.3) (layer "F.Cu") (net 10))
 (segment (start 147.6 62.65) (end 141.38 68.87) (width 0.3) (layer "F.Cu") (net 10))
 (segment (start 147.6 61.9) (end 147.6 62.65) (width 0.3) (layer "F.Cu") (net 10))
 (segment (start 149.2875 59.9) (end 150.1 59.0875) (width 0.3) (layer "F.Cu") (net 1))
 (segment (start 147.6 59.9) (end 149.2875 59.9) (width 0.3) (layer "F.Cu") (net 1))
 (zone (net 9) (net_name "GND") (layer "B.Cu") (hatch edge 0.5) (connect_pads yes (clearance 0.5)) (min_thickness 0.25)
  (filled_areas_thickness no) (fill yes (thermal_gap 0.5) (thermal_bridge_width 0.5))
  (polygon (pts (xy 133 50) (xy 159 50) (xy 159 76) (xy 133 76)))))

